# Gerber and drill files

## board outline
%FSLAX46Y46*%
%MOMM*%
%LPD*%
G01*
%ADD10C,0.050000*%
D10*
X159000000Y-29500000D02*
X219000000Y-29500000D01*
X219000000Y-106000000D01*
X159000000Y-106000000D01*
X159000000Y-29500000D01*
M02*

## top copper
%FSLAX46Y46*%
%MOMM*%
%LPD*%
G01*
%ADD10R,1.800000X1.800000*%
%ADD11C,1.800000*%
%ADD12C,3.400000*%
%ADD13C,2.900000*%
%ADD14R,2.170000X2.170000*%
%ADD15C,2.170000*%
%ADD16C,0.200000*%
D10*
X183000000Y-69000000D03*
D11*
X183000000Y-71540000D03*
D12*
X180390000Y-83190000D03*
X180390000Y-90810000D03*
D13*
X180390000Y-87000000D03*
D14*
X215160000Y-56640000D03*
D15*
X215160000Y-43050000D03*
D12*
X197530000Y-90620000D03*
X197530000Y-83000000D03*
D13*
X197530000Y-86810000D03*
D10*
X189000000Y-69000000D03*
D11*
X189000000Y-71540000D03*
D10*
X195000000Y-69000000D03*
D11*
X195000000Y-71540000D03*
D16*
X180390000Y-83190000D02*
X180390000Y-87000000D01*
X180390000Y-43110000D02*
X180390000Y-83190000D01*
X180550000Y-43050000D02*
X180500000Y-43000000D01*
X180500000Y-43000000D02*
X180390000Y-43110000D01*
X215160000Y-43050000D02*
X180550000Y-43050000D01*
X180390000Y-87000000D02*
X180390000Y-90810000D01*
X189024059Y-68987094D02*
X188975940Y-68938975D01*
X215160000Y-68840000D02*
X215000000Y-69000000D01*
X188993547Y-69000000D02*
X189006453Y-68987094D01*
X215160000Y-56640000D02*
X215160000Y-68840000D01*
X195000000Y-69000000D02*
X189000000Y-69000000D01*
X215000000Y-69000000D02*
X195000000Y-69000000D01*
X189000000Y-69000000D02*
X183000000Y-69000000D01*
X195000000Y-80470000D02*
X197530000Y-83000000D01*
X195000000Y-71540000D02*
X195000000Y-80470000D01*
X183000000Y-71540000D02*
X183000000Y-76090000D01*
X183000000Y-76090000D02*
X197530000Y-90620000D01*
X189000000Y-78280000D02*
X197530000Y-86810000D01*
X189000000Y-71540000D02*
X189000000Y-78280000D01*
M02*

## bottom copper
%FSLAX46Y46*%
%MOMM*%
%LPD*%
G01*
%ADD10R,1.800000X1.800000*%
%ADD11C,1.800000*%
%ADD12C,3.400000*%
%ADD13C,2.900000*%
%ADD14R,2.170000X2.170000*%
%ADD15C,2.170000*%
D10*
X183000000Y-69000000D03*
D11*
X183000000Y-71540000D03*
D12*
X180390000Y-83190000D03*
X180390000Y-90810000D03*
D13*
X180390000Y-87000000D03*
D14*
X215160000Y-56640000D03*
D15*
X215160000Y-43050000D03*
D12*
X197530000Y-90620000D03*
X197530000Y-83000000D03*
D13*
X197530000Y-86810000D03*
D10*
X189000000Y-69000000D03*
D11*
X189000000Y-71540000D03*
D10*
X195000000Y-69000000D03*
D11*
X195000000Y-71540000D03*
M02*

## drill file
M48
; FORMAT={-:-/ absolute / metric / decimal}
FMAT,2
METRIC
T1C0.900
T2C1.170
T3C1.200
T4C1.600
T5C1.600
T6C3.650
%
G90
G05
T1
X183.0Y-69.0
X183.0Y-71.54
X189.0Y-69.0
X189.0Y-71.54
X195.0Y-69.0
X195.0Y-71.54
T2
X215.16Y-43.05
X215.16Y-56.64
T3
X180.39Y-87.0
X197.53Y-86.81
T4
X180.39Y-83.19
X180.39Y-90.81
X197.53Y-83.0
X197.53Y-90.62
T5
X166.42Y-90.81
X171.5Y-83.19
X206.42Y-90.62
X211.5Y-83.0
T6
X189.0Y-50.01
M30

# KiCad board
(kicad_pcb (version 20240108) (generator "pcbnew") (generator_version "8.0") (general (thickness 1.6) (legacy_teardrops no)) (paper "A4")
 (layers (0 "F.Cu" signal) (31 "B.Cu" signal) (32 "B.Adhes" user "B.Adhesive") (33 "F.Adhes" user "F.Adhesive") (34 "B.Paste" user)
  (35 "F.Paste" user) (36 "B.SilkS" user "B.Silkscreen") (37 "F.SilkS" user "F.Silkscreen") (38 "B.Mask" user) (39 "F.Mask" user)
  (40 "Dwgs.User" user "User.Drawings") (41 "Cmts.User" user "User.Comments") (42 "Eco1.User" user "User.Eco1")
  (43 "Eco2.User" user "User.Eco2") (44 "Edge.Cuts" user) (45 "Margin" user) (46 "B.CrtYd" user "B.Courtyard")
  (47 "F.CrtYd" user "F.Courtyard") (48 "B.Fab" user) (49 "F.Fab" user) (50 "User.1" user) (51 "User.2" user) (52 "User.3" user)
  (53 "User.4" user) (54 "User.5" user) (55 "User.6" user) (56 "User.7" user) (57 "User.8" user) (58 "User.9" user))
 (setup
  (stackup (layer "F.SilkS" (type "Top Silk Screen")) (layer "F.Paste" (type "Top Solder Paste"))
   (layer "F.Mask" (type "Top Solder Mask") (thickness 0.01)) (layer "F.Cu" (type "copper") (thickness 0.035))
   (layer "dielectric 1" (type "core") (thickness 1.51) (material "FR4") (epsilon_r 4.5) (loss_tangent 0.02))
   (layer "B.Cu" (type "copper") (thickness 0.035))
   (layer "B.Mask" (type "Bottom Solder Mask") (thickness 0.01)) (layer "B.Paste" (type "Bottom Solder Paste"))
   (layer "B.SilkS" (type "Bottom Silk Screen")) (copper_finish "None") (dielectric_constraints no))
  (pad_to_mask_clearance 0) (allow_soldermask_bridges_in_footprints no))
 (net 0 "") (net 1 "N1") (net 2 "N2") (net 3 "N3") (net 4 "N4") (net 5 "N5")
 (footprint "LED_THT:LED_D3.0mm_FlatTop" (layer "F.Cu") (at 183 69 -90)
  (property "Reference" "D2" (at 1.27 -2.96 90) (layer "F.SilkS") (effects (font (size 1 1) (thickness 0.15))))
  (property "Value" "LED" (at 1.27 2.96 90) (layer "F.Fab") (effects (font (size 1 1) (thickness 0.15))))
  (pad "1" thru_hole rect (at 0 0 270) (size 1.8 1.8) (drill 0.9) (layers "*.Cu" "*.Mask") (remove_unused_layers no) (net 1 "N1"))
  (pad "2" thru_hole circle (at 2.54 0 270) (size 1.8 1.8) (drill 0.9) (layers "*.Cu" "*.Mask") (remove_unused_layers no) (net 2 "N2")))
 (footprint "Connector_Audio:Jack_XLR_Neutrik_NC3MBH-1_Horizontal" (layer "F.Cu") (at 180.39 83.19 -90)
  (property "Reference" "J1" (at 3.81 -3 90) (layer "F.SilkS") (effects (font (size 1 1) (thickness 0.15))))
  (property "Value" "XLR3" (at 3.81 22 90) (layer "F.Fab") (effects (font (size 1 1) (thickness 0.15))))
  (pad "" np_thru_hole circle (at 0 8.89 270) (size 1.6 1.6) (drill 1.6) (layers "*.Cu" "*.Mask"))
  (pad "" np_thru_hole circle (at 7.62 13.97 270) (size 1.6 1.6) (drill 1.6) (layers "*.Cu" "*.Mask"))
  (pad "1" thru_hole circle (at 0 0 270) (size 3.4 3.4) (drill 1.6) (layers "*.Cu" "*.Mask") (remove_unused_layers no) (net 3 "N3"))
  (pad "2" thru_hole circle (at 7.62 0 270) (size 3.4 3.4) (drill 1.6) (layers "*.Cu" "*.Mask") (remove_unused_layers no) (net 3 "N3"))
  (pad "3" thru_hole circle (at 3.81 0 270) (size 2.9 2.9) (drill 1.2) (layers "*.Cu" "*.Mask") (remove_unused_layers no) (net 3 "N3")))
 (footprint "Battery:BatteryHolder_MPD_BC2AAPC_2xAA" (layer "F.Cu") (at 215.16 56.64 180)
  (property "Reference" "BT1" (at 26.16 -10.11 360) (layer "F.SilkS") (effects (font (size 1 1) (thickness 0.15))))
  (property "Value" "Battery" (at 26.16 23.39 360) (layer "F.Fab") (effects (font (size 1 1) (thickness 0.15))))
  (pad "" np_thru_hole circle (at 26.16 6.63 180) (size 3.65 3.65) (drill 3.65) (layers "*.Cu" "*.Mask"))
  (pad "1" thru_hole rect (at 0 0 180) (size 2.17 2.17) (drill 1.17) (layers "*.Cu" "*.Mask") (remove_unused_layers no) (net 1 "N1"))
  (pad "2" thru_hole circle (at 0 13.59 180) (size 2.17 2.17) (drill 1.17) (layers "*.Cu" "*.Mask") (remove_unused_layers no) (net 3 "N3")))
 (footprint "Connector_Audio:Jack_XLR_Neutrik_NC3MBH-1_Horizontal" (layer "F.Cu") (at 197.53 90.62 90)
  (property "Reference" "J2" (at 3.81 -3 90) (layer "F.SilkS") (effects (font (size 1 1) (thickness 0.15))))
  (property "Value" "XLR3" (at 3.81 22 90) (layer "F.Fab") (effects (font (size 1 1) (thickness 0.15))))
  (pad "" np_thru_hole circle (at 0 8.89 90) (size 1.6 1.6) (drill 1.6) (layers "*.Cu" "*.Mask"))
  (pad "" np_thru_hole circle (at 7.62 13.97 90) (size 1.6 1.6) (drill 1.6) (layers "*.Cu" "*.Mask"))
  (pad "1" thru_hole circle (at 0 0 90) (size 3.4 3.4) (drill 1.6) (layers "*.Cu" "*.Mask") (remove_unused_layers no) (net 2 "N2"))
  (pad "2" thru_hole circle (at 7.62 0 90) (size 3.4 3.4) (drill 1.6) (layers "*.Cu" "*.Mask") (remove_unused_layers no) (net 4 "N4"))
  (pad "3" thru_hole circle (at 3.81 0 90) (size 2.9 2.9) (drill 1.2) (layers "*.Cu" "*.Mask") (remove_unused_layers no) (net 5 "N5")))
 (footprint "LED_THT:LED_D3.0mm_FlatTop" (layer "F.Cu") (at 189 69 -90)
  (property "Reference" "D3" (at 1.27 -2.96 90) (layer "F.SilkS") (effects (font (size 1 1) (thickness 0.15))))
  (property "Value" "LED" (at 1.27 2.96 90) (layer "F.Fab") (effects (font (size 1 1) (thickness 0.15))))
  (pad "1" thru_hole rect (at 0 0 270) (size 1.8 1.8) (drill 0.9) (layers "*.Cu" "*.Mask") (remove_unused_layers no) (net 1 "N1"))
  (pad "2" thru_hole circle (at 2.54 0 270) (size 1.8 1.8) (drill 0.9) (layers "*.Cu" "*.Mask") (remove_unused_layers no) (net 5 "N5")))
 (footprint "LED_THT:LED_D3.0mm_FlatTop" (layer "F.Cu") (at 195 69 -90)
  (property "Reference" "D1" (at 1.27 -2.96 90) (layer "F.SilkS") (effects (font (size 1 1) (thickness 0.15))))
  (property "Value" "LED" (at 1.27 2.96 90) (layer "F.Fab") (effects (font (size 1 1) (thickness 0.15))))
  (pad "1" thru_hole rect (at 0 0 270) (size 1.8 1.8) (drill 0.9) (layers "*.Cu" "*.Mask") (remove_unused_layers no) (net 1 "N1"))
  (pad "2" thru_hole circle (at 2.54 0 270) (size 1.8 1.8) (drill 0.9) (layers "*.Cu" "*.Mask") (remove_unused_layers no) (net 4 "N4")))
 (gr_rect (start 159 29.5) (end 219 106) (stroke (width 0.05) (type default)) (fill none) (layer "Edge.Cuts"))
 (segment (start 180.39 83.19) (end 180.39 87) (width 0.2) (layer "F.Cu") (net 3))
 (segment (start 180.39 43.11) (end 180.39 83.19) (width 0.2) (layer "F.Cu") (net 3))
 (segment (start 180.55 43.05) (end 180.5 43) (width 0.2) (layer "F.Cu") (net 3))
 (segment (start 180.5 43) (end 180.39 43.11) (width 0.2) (layer "F.Cu") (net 3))
 (segment (start 215.16 43.05) (end 180.55 43.05) (width 0.2) (layer "F.Cu") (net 3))
 (segment (start 180.39 87) (end 180.39 90.81) (width 0.2) (layer "F.Cu") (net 3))
 (segment (start 189.024059 68.987094) (end 188.97594 68.938975) (width 0.2) (layer "F.Cu") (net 1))
 (segment (start 215.16 68.84) (end 215 69) (width 0.2) (layer "F.Cu") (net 1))
 (segment (start 188.993547 69) (end 189.006453 68.987094) (width 0.2) (layer "F.Cu") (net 1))
 (segment (start 215.16 56.64) (end 215.16 68.84) (width 0.2) (layer "F.Cu") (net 1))
 (segment (start 195 69) (end 189 69) (width 0.2) (layer "F.Cu") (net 1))
 (segment (start 215 69) (end 195 69) (width 0.2) (layer "F.Cu") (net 1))
 (segment (start 189 69) (end 183 69) (width 0.2) (layer "F.Cu") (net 1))
 (segment (start 195 80.47) (end 197.53 83) (width 0.2) (layer "F.Cu") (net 4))
 (segment (start 195 71.54) (end 195 80.47) (width 0.2) (layer "F.Cu") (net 4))
 (segment (start 183 71.54) (end 183 76.09) (width 0.2) (layer "F.Cu") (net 2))
 (segment (start 183 76.09) (end 197.53 90.62) (width 0.2) (layer "F.Cu") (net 2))
 (segment (start 189 78.28) (end 197.53 86.81) (width 0.2) (layer "F.Cu") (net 5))
 (segment (start 189 71.54) (end 189 78.28) (width 0.2) (layer "F.Cu") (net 5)))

